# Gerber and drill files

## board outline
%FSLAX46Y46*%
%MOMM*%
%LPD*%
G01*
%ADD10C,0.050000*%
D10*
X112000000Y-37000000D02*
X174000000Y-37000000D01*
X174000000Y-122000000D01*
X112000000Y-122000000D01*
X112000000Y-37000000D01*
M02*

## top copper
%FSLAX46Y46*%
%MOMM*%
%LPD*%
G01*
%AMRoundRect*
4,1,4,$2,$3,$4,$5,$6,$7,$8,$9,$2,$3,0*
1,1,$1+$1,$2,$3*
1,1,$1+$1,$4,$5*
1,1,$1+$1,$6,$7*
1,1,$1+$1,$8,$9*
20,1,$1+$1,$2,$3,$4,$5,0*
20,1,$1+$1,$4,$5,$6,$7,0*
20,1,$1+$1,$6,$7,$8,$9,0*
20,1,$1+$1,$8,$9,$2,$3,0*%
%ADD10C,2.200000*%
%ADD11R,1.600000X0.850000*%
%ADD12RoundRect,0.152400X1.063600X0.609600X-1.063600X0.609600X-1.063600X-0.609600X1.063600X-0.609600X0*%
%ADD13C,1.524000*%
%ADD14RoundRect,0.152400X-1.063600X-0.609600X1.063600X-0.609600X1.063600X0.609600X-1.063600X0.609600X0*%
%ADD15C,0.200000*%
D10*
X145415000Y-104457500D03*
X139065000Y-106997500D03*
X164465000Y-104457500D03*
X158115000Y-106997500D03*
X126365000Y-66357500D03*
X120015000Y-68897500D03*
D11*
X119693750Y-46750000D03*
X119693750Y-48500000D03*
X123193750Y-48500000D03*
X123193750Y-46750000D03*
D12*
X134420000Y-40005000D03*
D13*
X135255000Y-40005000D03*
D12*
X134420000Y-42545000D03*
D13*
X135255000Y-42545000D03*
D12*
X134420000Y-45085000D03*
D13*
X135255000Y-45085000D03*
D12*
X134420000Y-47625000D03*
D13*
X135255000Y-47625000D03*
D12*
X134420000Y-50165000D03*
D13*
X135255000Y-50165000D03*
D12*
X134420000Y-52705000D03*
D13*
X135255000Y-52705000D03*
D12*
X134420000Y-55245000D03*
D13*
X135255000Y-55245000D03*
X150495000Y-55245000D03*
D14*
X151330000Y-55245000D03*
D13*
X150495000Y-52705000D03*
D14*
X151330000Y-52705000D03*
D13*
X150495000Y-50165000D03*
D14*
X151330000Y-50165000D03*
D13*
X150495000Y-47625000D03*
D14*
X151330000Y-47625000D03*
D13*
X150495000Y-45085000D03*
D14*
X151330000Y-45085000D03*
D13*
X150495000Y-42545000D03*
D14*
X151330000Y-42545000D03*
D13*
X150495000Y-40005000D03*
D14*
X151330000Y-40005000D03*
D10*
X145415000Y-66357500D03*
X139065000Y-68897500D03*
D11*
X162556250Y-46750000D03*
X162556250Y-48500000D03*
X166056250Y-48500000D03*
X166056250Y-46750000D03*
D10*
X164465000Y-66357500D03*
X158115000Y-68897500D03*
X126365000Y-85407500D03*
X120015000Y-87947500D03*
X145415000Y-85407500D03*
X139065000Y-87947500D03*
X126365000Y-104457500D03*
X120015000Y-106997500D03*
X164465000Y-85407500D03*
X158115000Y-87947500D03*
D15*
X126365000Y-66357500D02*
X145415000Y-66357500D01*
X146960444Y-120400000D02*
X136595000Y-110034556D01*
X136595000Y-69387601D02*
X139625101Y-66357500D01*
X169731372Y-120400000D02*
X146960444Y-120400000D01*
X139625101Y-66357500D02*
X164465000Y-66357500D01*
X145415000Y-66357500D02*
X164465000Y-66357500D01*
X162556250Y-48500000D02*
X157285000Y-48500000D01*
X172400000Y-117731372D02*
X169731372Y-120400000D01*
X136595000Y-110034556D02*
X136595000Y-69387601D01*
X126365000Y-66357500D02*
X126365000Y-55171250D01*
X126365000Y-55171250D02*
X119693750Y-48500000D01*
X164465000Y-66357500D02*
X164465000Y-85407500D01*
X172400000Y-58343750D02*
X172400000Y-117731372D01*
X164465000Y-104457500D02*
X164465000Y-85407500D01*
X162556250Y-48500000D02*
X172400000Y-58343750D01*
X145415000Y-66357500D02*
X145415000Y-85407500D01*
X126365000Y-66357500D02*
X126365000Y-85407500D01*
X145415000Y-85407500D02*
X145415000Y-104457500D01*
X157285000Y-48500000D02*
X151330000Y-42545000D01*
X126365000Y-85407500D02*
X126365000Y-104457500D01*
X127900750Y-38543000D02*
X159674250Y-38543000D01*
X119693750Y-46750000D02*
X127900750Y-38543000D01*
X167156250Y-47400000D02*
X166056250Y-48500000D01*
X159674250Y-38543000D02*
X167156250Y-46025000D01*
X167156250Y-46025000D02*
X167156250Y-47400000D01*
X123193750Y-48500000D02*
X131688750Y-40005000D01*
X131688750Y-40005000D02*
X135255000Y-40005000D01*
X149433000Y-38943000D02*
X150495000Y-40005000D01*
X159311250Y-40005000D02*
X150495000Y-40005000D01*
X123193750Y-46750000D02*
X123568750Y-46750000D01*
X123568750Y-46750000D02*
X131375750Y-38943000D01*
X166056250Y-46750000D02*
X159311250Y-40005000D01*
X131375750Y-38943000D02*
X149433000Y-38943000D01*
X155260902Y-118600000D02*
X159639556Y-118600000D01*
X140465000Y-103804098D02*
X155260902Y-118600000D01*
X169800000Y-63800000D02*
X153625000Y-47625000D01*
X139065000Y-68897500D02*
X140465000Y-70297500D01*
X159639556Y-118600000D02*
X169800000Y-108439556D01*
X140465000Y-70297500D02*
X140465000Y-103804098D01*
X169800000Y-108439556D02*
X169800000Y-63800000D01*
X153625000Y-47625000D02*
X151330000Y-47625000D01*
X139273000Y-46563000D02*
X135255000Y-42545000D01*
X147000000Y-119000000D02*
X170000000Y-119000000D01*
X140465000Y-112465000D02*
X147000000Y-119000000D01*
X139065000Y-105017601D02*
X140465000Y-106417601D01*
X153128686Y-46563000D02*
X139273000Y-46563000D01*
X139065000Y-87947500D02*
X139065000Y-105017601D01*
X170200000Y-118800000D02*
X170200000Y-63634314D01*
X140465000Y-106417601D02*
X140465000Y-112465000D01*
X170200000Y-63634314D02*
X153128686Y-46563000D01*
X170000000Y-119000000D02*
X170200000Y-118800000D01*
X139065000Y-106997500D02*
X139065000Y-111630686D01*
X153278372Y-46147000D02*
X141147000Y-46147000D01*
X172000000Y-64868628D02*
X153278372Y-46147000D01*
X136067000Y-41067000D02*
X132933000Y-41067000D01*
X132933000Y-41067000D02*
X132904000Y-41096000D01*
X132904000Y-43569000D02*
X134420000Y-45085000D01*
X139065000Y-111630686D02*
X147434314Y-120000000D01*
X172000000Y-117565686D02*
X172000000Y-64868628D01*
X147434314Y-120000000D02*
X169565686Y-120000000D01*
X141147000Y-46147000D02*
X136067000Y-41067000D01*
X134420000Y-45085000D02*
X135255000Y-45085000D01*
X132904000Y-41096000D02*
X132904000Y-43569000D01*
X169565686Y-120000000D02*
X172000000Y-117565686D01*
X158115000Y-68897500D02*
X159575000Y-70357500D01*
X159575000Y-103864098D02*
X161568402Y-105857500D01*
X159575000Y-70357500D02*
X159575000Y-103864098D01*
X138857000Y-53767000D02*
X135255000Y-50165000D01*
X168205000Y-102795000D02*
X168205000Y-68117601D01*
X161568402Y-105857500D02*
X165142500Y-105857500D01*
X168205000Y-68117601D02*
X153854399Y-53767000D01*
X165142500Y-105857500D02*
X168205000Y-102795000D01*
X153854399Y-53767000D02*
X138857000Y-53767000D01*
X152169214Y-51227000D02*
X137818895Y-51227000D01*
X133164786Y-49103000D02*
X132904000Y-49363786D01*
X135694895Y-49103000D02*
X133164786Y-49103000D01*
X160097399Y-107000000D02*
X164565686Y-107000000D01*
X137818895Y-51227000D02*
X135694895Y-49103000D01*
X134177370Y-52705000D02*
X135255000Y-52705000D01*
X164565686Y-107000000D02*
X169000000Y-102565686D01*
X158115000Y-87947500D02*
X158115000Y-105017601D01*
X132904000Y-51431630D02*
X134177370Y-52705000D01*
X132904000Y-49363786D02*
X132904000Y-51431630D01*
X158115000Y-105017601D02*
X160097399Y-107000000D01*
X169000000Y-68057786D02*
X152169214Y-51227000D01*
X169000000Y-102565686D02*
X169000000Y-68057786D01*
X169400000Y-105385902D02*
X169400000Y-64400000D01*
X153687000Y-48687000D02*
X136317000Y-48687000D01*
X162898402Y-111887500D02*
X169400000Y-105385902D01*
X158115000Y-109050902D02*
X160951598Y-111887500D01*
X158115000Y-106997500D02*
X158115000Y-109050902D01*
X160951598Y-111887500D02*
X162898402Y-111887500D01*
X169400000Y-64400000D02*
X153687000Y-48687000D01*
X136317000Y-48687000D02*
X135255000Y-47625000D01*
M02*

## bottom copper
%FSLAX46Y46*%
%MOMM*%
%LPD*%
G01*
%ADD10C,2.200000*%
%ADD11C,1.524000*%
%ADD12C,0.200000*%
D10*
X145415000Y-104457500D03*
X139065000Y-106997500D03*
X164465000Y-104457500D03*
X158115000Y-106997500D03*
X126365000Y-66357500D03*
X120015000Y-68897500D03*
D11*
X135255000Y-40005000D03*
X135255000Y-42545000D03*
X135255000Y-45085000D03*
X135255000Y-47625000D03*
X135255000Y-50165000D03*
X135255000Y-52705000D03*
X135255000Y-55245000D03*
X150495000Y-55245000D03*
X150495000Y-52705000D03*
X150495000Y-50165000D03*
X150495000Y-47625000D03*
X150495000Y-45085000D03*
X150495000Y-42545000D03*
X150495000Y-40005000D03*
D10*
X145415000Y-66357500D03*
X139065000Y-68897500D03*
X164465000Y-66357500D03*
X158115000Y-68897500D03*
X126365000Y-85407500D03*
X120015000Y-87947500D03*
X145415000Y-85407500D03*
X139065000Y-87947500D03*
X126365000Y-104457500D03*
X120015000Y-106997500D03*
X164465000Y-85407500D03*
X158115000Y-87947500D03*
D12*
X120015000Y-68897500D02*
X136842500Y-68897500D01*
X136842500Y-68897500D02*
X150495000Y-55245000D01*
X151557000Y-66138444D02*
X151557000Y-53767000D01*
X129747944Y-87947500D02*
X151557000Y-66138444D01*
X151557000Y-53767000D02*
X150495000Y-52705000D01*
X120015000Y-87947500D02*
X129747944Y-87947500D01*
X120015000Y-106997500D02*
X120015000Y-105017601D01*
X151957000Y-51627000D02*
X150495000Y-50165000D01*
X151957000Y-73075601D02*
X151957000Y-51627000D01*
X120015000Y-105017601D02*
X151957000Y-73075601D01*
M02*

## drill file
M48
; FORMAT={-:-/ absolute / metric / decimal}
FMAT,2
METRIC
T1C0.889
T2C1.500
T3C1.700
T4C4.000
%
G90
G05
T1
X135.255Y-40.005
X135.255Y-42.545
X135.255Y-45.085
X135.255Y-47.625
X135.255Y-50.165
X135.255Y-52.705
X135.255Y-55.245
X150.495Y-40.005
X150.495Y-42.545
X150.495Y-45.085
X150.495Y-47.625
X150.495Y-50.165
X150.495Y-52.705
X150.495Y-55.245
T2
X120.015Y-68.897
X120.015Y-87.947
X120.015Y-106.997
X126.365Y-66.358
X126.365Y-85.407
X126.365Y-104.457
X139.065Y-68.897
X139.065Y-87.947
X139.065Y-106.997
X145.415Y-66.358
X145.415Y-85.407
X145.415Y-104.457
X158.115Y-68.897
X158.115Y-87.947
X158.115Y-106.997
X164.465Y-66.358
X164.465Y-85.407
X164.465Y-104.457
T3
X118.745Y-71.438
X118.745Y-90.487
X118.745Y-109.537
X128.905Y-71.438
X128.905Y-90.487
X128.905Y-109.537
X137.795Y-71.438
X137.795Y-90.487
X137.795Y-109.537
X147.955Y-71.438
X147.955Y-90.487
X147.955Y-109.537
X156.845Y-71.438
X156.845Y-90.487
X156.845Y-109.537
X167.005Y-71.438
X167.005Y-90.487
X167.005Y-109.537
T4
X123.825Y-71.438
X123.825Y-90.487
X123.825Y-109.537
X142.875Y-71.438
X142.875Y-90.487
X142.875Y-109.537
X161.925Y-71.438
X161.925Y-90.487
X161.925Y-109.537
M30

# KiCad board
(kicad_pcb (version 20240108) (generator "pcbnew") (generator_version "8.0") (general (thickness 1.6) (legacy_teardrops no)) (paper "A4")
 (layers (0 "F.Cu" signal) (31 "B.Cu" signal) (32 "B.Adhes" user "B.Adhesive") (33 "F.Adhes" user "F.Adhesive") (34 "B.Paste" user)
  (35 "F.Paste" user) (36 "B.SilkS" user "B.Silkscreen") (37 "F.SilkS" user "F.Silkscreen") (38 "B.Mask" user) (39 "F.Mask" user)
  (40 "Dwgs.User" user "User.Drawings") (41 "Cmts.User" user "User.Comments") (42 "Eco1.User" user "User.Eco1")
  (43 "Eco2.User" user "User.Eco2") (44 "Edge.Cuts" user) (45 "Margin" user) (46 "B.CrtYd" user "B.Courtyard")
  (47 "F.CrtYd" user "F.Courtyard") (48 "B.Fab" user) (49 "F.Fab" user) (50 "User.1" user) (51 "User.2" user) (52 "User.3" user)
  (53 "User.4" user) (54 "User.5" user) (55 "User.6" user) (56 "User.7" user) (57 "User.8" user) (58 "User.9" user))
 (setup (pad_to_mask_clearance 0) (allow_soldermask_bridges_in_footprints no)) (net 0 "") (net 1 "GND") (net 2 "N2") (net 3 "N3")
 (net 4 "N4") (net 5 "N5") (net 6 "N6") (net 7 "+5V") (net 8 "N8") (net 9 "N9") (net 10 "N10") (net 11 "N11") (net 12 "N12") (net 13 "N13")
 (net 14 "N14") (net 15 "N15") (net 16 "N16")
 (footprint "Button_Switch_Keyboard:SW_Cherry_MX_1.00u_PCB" (layer "F.Cu") (at 145.415 104.4575)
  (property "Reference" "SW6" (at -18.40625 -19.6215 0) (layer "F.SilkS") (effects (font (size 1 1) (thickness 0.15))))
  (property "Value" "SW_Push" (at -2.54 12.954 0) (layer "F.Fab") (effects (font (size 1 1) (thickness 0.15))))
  (pad "" np_thru_hole circle (at -7.62 5.08) (size 1.7 1.7) (drill 1.7) (layers "*.Cu" "*.Mask"))
  (pad "" np_thru_hole circle (at -2.54 5.08) (size 4 4) (drill 4) (layers "*.Cu" "*.Mask"))
  (pad "" np_thru_hole circle (at 2.54 5.08) (size 1.7 1.7) (drill 1.7) (layers "*.Cu" "*.Mask"))
  (pad "1" thru_hole circle (at 0 0) (size 2.2 2.2) (drill 1.5) (layers "*.Cu" "*.Mask") (remove_unused_layers no) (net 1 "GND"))
  (pad "2" thru_hole circle (at -6.35 2.54) (size 2.2 2.2) (drill 1.5) (layers "*.Cu" "*.Mask") (remove_unused_layers no) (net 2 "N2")))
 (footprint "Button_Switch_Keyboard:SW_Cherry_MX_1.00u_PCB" (layer "F.Cu") (at 164.465 104.4575)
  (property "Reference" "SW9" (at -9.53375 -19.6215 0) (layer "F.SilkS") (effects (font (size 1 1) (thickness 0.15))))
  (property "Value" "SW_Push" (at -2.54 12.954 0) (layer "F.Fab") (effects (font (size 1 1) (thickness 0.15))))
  (pad "" np_thru_hole circle (at -7.62 5.08) (size 1.7 1.7) (drill 1.7) (layers "*.Cu" "*.Mask"))
  (pad "" np_thru_hole circle (at -2.54 5.08) (size 4 4) (drill 4) (layers "*.Cu" "*.Mask"))
  (pad "" np_thru_hole circle (at 2.54 5.08) (size 1.7 1.7) (drill 1.7) (layers "*.Cu" "*.Mask"))
  (pad "1" thru_hole circle (at 0 0) (size 2.2 2.2) (drill 1.5) (layers "*.Cu" "*.Mask") (remove_unused_layers no) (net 1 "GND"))
  (pad "2" thru_hole circle (at -6.35 2.54) (size 2.2 2.2) (drill 1.5) (layers "*.Cu" "*.Mask") (remove_unused_layers no) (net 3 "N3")))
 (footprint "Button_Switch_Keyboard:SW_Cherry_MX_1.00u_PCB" (layer "F.Cu") (at 126.365 66.3575)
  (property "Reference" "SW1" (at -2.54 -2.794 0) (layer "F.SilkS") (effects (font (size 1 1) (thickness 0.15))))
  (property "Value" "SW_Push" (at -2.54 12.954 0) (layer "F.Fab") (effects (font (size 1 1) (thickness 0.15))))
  (pad "" np_thru_hole circle (at -7.62 5.08) (size 1.7 1.7) (drill 1.7) (layers "*.Cu" "*.Mask"))
  (pad "" np_thru_hole circle (at -2.54 5.08) (size 4 4) (drill 4) (layers "*.Cu" "*.Mask"))
  (pad "" np_thru_hole circle (at 2.54 5.08) (size 1.7 1.7) (drill 1.7) (layers "*.Cu" "*.Mask"))
  (pad "1" thru_hole circle (at 0 0) (size 2.2 2.2) (drill 1.5) (layers "*.Cu" "*.Mask") (remove_unused_layers no) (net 1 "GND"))
  (pad "2" thru_hole circle (at -6.35 2.54) (size 2.2 2.2) (drill 1.5) (layers "*.Cu" "*.Mask") (remove_unused_layers no) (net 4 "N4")))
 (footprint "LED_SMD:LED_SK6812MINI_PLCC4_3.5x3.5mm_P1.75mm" (layer "F.Cu") (at 121.44375 47.625)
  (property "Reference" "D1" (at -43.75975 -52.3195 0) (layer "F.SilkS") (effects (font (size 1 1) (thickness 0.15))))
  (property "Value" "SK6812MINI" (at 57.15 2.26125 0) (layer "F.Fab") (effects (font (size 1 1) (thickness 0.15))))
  (pad "1" smd rect (at -1.75 -0.875) (size 1.6 0.85) (layers "F.Cu" "F.Paste" "F.Mask") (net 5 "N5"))
  (pad "2" smd rect (at -1.75 0.875) (size 1.6 0.85) (layers "F.Cu" "F.Paste" "F.Mask") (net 1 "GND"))
  (pad "3" smd rect (at 1.75 0.875) (size 1.6 0.85) (layers "F.Cu" "F.Paste" "F.Mask") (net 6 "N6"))
  (pad "4" smd rect (at 1.75 -0.875) (size 1.6 0.85) (layers "F.Cu" "F.Paste" "F.Mask") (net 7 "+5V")))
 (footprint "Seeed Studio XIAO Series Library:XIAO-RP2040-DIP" (layer "F.Cu") (at 142.875 47.625)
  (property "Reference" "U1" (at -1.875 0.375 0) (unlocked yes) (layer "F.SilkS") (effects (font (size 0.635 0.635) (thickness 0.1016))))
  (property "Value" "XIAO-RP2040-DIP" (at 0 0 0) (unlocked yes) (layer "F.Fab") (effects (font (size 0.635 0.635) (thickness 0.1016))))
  (pad "1" smd roundrect (at -8.455 -7.62 180) (size 2.432 1.524) (layers "F.Cu" "F.Mask") (roundrect_rratio 0.1) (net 6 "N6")
   (thermal_bridge_angle 45))
  (pad "1" thru_hole circle (at -7.62 -7.62 180) (size 1.524 1.524) (drill 0.889) (layers "*.Cu" "*.Mask") (remove_unused_layers no)
   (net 6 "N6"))
  (pad "2" smd roundrect (at -8.455 -5.08 180) (size 2.432 1.524) (layers "F.Cu" "F.Mask") (roundrect_rratio 0.1) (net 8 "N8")
   (thermal_bridge_angle 45))
  (pad "2" thru_hole circle (at -7.62 -5.08 180) (size 1.524 1.524) (drill 0.889) (layers "*.Cu" "*.Mask") (remove_unused_layers no)
   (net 8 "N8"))
  (pad "3" smd roundrect (at -8.455 -2.54 180) (size 2.432 1.524) (layers "F.Cu" "F.Mask") (roundrect_rratio 0.1) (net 2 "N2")
   (thermal_bridge_angle 45))
  (pad "3" thru_hole circle (at -7.62 -2.54 180) (size 1.524 1.524) (drill 0.889) (layers "*.Cu" "*.Mask") (remove_unused_layers no)
   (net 2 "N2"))
  (pad "4" smd roundrect (at -8.455 0 180) (size 2.432 1.524) (layers "F.Cu" "F.Mask") (roundrect_rratio 0.1) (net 3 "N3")
   (thermal_bridge_angle 45))
  (pad "4" thru_hole circle (at -7.62 0 180) (size 1.524 1.524) (drill 0.889) (layers "*.Cu" "*.Mask") (remove_unused_layers no)
   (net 3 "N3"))
  (pad "5" smd roundrect (at -8.455 2.54 180) (size 2.432 1.524) (layers "F.Cu" "F.Mask") (roundrect_rratio 0.1) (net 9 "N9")
   (thermal_bridge_angle 45))
  (pad "5" thru_hole circle (at -7.62 2.54 180) (size 1.524 1.524) (drill 0.889) (layers "*.Cu" "*.Mask") (remove_unused_layers no)
   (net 9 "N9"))
  (pad "6" smd roundrect (at -8.455 5.08 180) (size 2.432 1.524) (layers "F.Cu" "F.Mask") (roundrect_rratio 0.1) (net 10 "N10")
   (thermal_bridge_angle 45))
  (pad "6" thru_hole circle (at -7.62 5.08 180) (size 1.524 1.524) (drill 0.889) (layers "*.Cu" "*.Mask") (remove_unused_layers no)
   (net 10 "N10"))
  (pad "7" smd roundrect (at -8.455 7.62 180) (size 2.432 1.524) (layers "F.Cu" "F.Mask") (roundrect_rratio 0.1) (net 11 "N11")
   (thermal_bridge_angle 45))
  (pad "7" thru_hole circle (at -7.62 7.62 180) (size 1.524 1.524) (drill 0.889) (layers "*.Cu" "*.Mask") (remove_unused_layers no)
   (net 11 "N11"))
  (pad "8" thru_hole circle (at 7.62 7.62) (size 1.524 1.524) (drill 0.889) (layers "*.Cu" "*.Mask") (remove_unused_layers no) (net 4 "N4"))
  (pad "8" smd roundrect (at 8.455 7.62) (size 2.432 1.524) (layers "F.Cu" "F.Mask") (roundrect_rratio 0.1) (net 4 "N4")
   (thermal_bridge_angle 45))
  (pad "9" thru_hole circle (at 7.62 5.08) (size 1.524 1.524) (drill 0.889) (layers "*.Cu" "*.Mask") (remove_unused_layers no)
   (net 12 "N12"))
  (pad "9" smd roundrect (at 8.455 5.08) (size 2.432 1.524) (layers "F.Cu" "F.Mask") (roundrect_rratio 0.1) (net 12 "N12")
   (thermal_bridge_angle 45))
  (pad "10" thru_hole circle (at 7.62 2.54) (size 1.524 1.524) (drill 0.889) (layers "*.Cu" "*.Mask") (remove_unused_layers no)
   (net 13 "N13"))
  (pad "10" smd roundrect (at 8.455 2.54) (size 2.432 1.524) (layers "F.Cu" "F.Mask") (roundrect_rratio 0.1) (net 13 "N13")
   (thermal_bridge_angle 45))
  (pad "11" thru_hole circle (at 7.62 0) (size 1.524 1.524) (drill 0.889) (layers "*.Cu" "*.Mask") (remove_unused_layers no) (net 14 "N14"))
  (pad "11" smd roundrect (at 8.455 0) (size 2.432 1.524) (layers "F.Cu" "F.Mask") (roundrect_rratio 0.1) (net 14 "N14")
   (thermal_bridge_angle 45))
  (pad "12" thru_hole circle (at 7.62 -2.54) (size 1.524 1.524) (drill 0.889) (layers "*.Cu" "*.Mask") (remove_unused_layers no)
   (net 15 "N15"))
  (pad "12" smd roundrect (at 8.455 -2.54) (size 2.432 1.524) (layers "F.Cu" "F.Mask") (roundrect_rratio 0.1) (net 15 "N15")
   (thermal_bridge_angle 45))
  (pad "13" thru_hole circle (at 7.62 -5.08) (size 1.524 1.524) (drill 0.889) (layers "*.Cu" "*.Mask") (remove_unused_layers no)
   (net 1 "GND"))
  (pad "13" smd roundrect (at 8.455 -5.08) (size 2.432 1.524) (layers "F.Cu" "F.Mask") (roundrect_rratio 0.1) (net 1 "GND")
   (thermal_bridge_angle 45))
  (pad "14" thru_hole circle (at 7.62 -7.62) (size 1.524 1.524) (drill 0.889) (layers "*.Cu" "*.Mask") (remove_unused_layers no)
   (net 7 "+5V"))
  (pad "14" smd roundrect (at 8.455 -7.62) (size 2.432 1.524) (layers "F.Cu" "F.Mask") (roundrect_rratio 0.1) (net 7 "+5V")
   (thermal_bridge_angle 45)))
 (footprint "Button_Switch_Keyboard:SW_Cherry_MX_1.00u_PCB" (layer "F.Cu") (at 145.415 66.3575)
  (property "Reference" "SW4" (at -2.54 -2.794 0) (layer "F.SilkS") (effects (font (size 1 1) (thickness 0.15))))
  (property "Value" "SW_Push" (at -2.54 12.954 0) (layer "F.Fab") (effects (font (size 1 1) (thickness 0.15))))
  (pad "" np_thru_hole circle (at -7.62 5.08) (size 1.7 1.7) (drill 1.7) (layers "*.Cu" "*.Mask"))
  (pad "" np_thru_hole circle (at -2.54 5.08) (size 4 4) (drill 4) (layers "*.Cu" "*.Mask"))
  (pad "" np_thru_hole circle (at 2.54 5.08) (size 1.7 1.7) (drill 1.7) (layers "*.Cu" "*.Mask"))
  (pad "1" thru_hole circle (at 0 0) (size 2.2 2.2) (drill 1.5) (layers "*.Cu" "*.Mask") (remove_unused_layers no) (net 1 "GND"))
  (pad "2" thru_hole circle (at -6.35 2.54) (size 2.2 2.2) (drill 1.5) (layers "*.Cu" "*.Mask") (remove_unused_layers no) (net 14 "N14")))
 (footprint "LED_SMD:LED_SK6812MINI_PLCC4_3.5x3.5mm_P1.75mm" (layer "F.Cu") (at 164.30625 47.625)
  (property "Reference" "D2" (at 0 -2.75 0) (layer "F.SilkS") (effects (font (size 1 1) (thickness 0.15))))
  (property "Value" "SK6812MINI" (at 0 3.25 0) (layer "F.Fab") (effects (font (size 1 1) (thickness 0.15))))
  (pad "1" smd rect (at -1.75 -0.875) (size 1.6 0.85) (layers "F.Cu" "F.Paste" "F.Mask") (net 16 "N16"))
  (pad "2" smd rect (at -1.75 0.875) (size 1.6 0.85) (layers "F.Cu" "F.Paste" "F.Mask") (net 1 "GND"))
  (pad "3" smd rect (at 1.75 0.875) (size 1.6 0.85) (layers "F.Cu" "F.Paste" "F.Mask") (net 5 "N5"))
  (pad "4" smd rect (at 1.75 -0.875) (size 1.6 0.85) (layers "F.Cu" "F.Paste" "F.Mask") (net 7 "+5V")))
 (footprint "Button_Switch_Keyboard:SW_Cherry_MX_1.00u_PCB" (layer "F.Cu") (at 164.465 66.3575)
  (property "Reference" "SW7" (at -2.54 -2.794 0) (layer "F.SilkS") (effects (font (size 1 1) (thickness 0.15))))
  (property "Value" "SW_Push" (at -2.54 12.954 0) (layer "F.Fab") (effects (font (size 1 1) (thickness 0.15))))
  (pad "" np_thru_hole circle (at -7.62 5.08) (size 1.7 1.7) (drill 1.7) (layers "*.Cu" "*.Mask"))
  (pad "" np_thru_hole circle (at -2.54 5.08) (size 4 4) (drill 4) (layers "*.Cu" "*.Mask"))
  (pad "" np_thru_hole circle (at 2.54 5.08) (size 1.7 1.7) (drill 1.7) (layers "*.Cu" "*.Mask"))
  (pad "1" thru_hole circle (at 0 0) (size 2.2 2.2) (drill 1.5) (layers "*.Cu" "*.Mask") (remove_unused_layers no) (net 1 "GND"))
  (pad "2" thru_hole circle (at -6.35 2.54) (size 2.2 2.2) (drill 1.5) (layers "*.Cu" "*.Mask") (remove_unused_layers no) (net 9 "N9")))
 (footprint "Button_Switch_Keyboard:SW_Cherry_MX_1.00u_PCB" (layer "F.Cu") (at 126.365 85.4075)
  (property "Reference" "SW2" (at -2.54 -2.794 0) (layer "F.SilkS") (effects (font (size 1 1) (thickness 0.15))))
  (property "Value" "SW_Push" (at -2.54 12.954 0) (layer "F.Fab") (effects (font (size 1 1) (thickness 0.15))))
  (pad "" np_thru_hole circle (at -7.62 5.08) (size 1.7 1.7) (drill 1.7) (layers "*.Cu" "*.Mask"))
  (pad "" np_thru_hole circle (at -2.54 5.08) (size 4 4) (drill 4) (layers "*.Cu" "*.Mask"))
  (pad "" np_thru_hole circle (at 2.54 5.08) (size 1.7 1.7) (drill 1.7) (layers "*.Cu" "*.Mask"))
  (pad "1" thru_hole circle (at 0 0) (size 2.2 2.2) (drill 1.5) (layers "*.Cu" "*.Mask") (remove_unused_layers no) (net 1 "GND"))
  (pad "2" thru_hole circle (at -6.35 2.54) (size 2.2 2.2) (drill 1.5) (layers "*.Cu" "*.Mask") (remove_unused_layers no) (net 12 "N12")))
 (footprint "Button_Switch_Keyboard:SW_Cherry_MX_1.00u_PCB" (layer "F.Cu") (at 145.415 85.4075)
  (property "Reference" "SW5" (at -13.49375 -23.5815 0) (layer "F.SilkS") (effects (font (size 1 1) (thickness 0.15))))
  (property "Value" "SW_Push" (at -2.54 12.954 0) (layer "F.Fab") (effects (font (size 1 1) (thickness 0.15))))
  (pad "" np_thru_hole circle (at -7.62 5.08) (size 1.7 1.7) (drill 1.7) (layers "*.Cu" "*.Mask"))
  (pad "" np_thru_hole circle (at -2.54 5.08) (size 4 4) (drill 4) (layers "*.Cu" "*.Mask"))
  (pad "" np_thru_hole circle (at 2.54 5.08) (size 1.7 1.7) (drill 1.7) (layers "*.Cu" "*.Mask"))
  (pad "1" thru_hole circle (at 0 0) (size 2.2 2.2) (drill 1.5) (layers "*.Cu" "*.Mask") (remove_unused_layers no) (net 1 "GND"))
  (pad "2" thru_hole circle (at -6.35 2.54) (size 2.2 2.2) (drill 1.5) (layers "*.Cu" "*.Mask") (remove_unused_layers no) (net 8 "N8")))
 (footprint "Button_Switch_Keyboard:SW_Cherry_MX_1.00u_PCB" (layer "F.Cu") (at 126.365 104.4575)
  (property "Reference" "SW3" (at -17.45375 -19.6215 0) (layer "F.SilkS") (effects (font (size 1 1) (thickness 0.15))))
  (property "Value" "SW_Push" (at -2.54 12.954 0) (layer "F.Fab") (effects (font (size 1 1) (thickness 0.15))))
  (pad "" np_thru_hole circle (at -7.62 5.08) (size 1.7 1.7) (drill 1.7) (layers "*.Cu" "*.Mask"))
  (pad "" np_thru_hole circle (at -2.54 5.08) (size 4 4) (drill 4) (layers "*.Cu" "*.Mask"))
  (pad "" np_thru_hole circle (at 2.54 5.08) (size 1.7 1.7) (drill 1.7) (layers "*.Cu" "*.Mask"))
  (pad "1" thru_hole circle (at 0 0) (size 2.2 2.2) (drill 1.5) (layers "*.Cu" "*.Mask") (remove_unused_layers no) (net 1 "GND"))
  (pad "2" thru_hole circle (at -6.35 2.54) (size 2.2 2.2) (drill 1.5) (layers "*.Cu" "*.Mask") (remove_unused_layers no) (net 13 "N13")))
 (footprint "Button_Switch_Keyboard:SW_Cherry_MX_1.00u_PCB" (layer "F.Cu") (at 164.465 85.4075)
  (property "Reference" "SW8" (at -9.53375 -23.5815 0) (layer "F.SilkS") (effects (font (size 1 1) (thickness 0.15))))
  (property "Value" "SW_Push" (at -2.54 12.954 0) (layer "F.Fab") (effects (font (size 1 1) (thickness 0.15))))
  (pad "" np_thru_hole circle (at -7.62 5.08) (size 1.7 1.7) (drill 1.7) (layers "*.Cu" "*.Mask"))
  (pad "" np_thru_hole circle (at -2.54 5.08) (size 4 4) (drill 4) (layers "*.Cu" "*.Mask"))
  (pad "" np_thru_hole circle (at 2.54 5.08) (size 1.7 1.7) (drill 1.7) (layers "*.Cu" "*.Mask"))
  (pad "1" thru_hole circle (at 0 0) (size 2.2 2.2) (drill 1.5) (layers "*.Cu" "*.Mask") (remove_unused_layers no) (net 1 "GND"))
  (pad "2" thru_hole circle (at -6.35 2.54) (size 2.2 2.2) (drill 1.5) (layers "*.Cu" "*.Mask") (remove_unused_layers no) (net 10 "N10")))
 (gr_rect (start 112 37) (end 174 122) (stroke (width 0.05) (type default)) (fill none) (layer "Edge.Cuts"))
 (segment (start 126.365 66.3575) (end 145.415 66.3575) (width 0.2) (layer "F.Cu") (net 1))
 (segment (start 146.960444 120.4) (end 136.595 110.034556) (width 0.2) (layer "F.Cu") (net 1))
 (segment (start 136.595 69.387601) (end 139.625101 66.3575) (width 0.2) (layer "F.Cu") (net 1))
 (segment (start 169.731372 120.4) (end 146.960444 120.4) (width 0.2) (layer "F.Cu") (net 1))
 (segment (start 139.625101 66.3575) (end 164.465 66.3575) (width 0.2) (layer "F.Cu") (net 1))
 (segment (start 145.415 66.3575) (end 164.465 66.3575) (width 0.2) (layer "F.Cu") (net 1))
 (segment (start 162.55625 48.5) (end 157.285 48.5) (width 0.2) (layer "F.Cu") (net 1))
 (segment (start 172.4 117.731372) (end 169.731372 120.4) (width 0.2) (layer "F.Cu") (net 1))
 (segment (start 136.595 110.034556) (end 136.595 69.387601) (width 0.2) (layer "F.Cu") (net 1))
 (segment (start 126.365 66.3575) (end 126.365 55.17125) (width 0.2) (layer "F.Cu") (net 1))
 (segment (start 126.365 55.17125) (end 119.69375 48.5) (width 0.2) (layer "F.Cu") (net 1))
 (segment (start 164.465 66.3575) (end 164.465 85.4075) (width 0.2) (layer "F.Cu") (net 1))
 (segment (start 172.4 58.34375) (end 172.4 117.731372) (width 0.2) (layer "F.Cu") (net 1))
 (segment (start 164.465 104.4575) (end 164.465 85.4075) (width 0.2) (layer "F.Cu") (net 1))
 (segment (start 162.55625 48.5) (end 172.4 58.34375) (width 0.2) (layer "F.Cu") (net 1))
 (segment (start 145.415 66.3575) (end 145.415 85.4075) (width 0.2) (layer "F.Cu") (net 1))
 (segment (start 126.365 66.3575) (end 126.365 85.4075) (width 0.2) (layer "F.Cu") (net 1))
 (segment (start 145.415 85.4075) (end 145.415 104.4575) (width 0.2) (layer "F.Cu") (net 1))
 (segment (start 157.285 48.5) (end 151.33 42.545) (width 0.2) (layer "F.Cu") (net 1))
 (segment (start 126.365 85.4075) (end 126.365 104.4575) (width 0.2) (layer "F.Cu") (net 1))
 (segment (start 127.90075 38.543) (end 159.67425 38.543) (width 0.2) (layer "F.Cu") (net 5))
 (segment (start 119.69375 46.75) (end 127.90075 38.543) (width 0.2) (layer "F.Cu") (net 5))
 (segment (start 167.15625 47.4) (end 166.05625 48.5) (width 0.2) (layer "F.Cu") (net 5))
 (segment (start 159.67425 38.543) (end 167.15625 46.025) (width 0.2) (layer "F.Cu") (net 5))
 (segment (start 167.15625 46.025) (end 167.15625 47.4) (width 0.2) (layer "F.Cu") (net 5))
 (segment (start 123.19375 48.5) (end 131.68875 40.005) (width 0.2) (layer "F.Cu") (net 6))
 (segment (start 131.68875 40.005) (end 135.255 40.005) (width 0.2) (layer "F.Cu") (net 6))
 (segment (start 149.433 38.943) (end 150.495 40.005) (width 0.2) (layer "F.Cu") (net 7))
 (segment (start 159.31125 40.005) (end 150.495 40.005) (width 0.2) (layer "F.Cu") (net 7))
 (segment (start 123.19375 46.75) (end 123.56875 46.75) (width 0.2) (layer "F.Cu") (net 7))
 (segment (start 123.56875 46.75) (end 131.37575 38.943) (width 0.2) (layer "F.Cu") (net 7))
 (segment (start 166.05625 46.75) (end 159.31125 40.005) (width 0.2) (layer "F.Cu") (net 7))
 (segment (start 131.37575 38.943) (end 149.433 38.943) (width 0.2) (layer "F.Cu") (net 7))
 (segment (start 120.015 68.8975) (end 136.8425 68.8975) (width 0.2) (layer "B.Cu") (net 4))
 (segment (start 136.8425 68.8975) (end 150.495 55.245) (width 0.2) (layer "B.Cu") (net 4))
 (segment (start 151.557 66.138444) (end 151.557 53.767) (width 0.2) (layer "B.Cu") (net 12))
 (segment (start 129.747944 87.9475) (end 151.557 66.138444) (width 0.2) (layer "B.Cu") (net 12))
 (segment (start 151.557 53.767) (end 150.495 52.705) (width 0.2) (layer "B.Cu") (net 12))
 (segment (start 120.015 87.9475) (end 129.747944 87.9475) (width 0.2) (layer "B.Cu") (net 12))
 (segment (start 120.015 106.9975) (end 120.015 105.017601) (width 0.2) (layer "B.Cu") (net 13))
 (segment (start 151.957 51.627) (end 150.495 50.165) (width 0.2) (layer "B.Cu") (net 13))
 (segment (start 151.957 73.075601) (end 151.957 51.627) (width 0.2) (layer "B.Cu") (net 13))
 (segment (start 120.015 105.017601) (end 151.957 73.075601) (width 0.2) (layer "B.Cu") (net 13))
 (segment (start 155.260902 118.6) (end 159.639556 118.6) (width 0.2) (layer "F.Cu") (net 14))
 (segment (start 140.465 103.804098) (end 155.260902 118.6) (width 0.2) (layer "F.Cu") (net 14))
 (segment (start 169.8 63.8) (end 153.625 47.625) (width 0.2) (layer "F.Cu") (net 14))
 (segment (start 139.065 68.8975) (end 140.465 70.2975) (width 0.2) (layer "F.Cu") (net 14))
 (segment (start 159.639556 118.6) (end 169.8 108.439556) (width 0.2) (layer "F.Cu") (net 14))
 (segment (start 140.465 70.2975) (end 140.465 103.804098) (width 0.2) (layer "F.Cu") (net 14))
 (segment (start 169.8 108.439556) (end 169.8 63.8) (width 0.2) (layer "F.Cu") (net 14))
 (segment (start 153.625 47.625) (end 151.33 47.625) (width 0.2) (layer "F.Cu") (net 14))
 (segment (start 139.273 46.563) (end 135.255 42.545) (width 0.2) (layer "F.Cu") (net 8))
 (segment (start 147 119) (end 170 119) (width 0.2) (layer "F.Cu") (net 8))
 (segment (start 140.465 112.465) (end 147 119) (width 0.2) (layer "F.Cu") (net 8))
 (segment (start 139.065 105.017601) (end 140.465 106.417601) (width 0.2) (layer "F.Cu") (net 8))
 (segment (start 153.128686 46.563) (end 139.273 46.563) (width 0.2) (layer "F.Cu") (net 8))
 (segment (start 139.065 87.9475) (end 139.065 105.017601) (width 0.2) (layer "F.Cu") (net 8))
 (segment (start 170.2 118.8) (end 170.2 63.634314) (width 0.2) (layer "F.Cu") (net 8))
 (segment (start 140.465 106.417601) (end 140.465 112.465) (width 0.2) (layer "F.Cu") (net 8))
 (segment (start 170.2 63.634314) (end 153.128686 46.563) (width 0.2) (layer "F.Cu") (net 8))
 (segment (start 170 119) (end 170.2 118.8) (width 0.2) (layer "F.Cu") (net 8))
 (segment (start 139.065 106.9975) (end 139.065 111.630686) (width 0.2) (layer "F.Cu") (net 2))
 (segment (start 153.278372 46.147) (end 141.147 46.147) (width 0.2) (layer "F.Cu") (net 2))
 (segment (start 172 64.868628) (end 153.278372 46.147) (width 0.2) (layer "F.Cu") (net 2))
 (segment (start 136.067 41.067) (end 132.933 41.067) (width 0.2) (layer "F.Cu") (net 2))
 (segment (start 132.933 41.067) (end 132.904 41.096) (width 0.2) (layer "F.Cu") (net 2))
 (segment (start 132.904 43.569) (end 134.42 45.085) (width 0.2) (layer "F.Cu") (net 2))
 (segment (start 139.065 111.630686) (end 147.434314 120) (width 0.2) (layer "F.Cu") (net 2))
 (segment (start 172 117.565686) (end 172 64.868628) (width 0.2) (layer "F.Cu") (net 2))
 (segment (start 147.434314 120) (end 169.565686 120) (width 0.2) (layer "F.Cu") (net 2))
 (segment (start 141.147 46.147) (end 136.067 41.067) (width 0.2) (layer "F.Cu") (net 2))
 (segment (start 134.42 45.085) (end 135.255 45.085) (width 0.2) (layer "F.Cu") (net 2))
 (segment (start 132.904 41.096) (end 132.904 43.569) (width 0.2) (layer "F.Cu") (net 2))
 (segment (start 169.565686 120) (end 172 117.565686) (width 0.2) (layer "F.Cu") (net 2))
 (segment (start 158.115 68.8975) (end 159.575 70.3575) (width 0.2) (layer "F.Cu") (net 9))
 (segment (start 159.575 103.864098) (end 161.568402 105.8575) (width 0.2) (layer "F.Cu") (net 9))
 (segment (start 159.575 70.3575) (end 159.575 103.864098) (width 0.2) (layer "F.Cu") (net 9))
 (segment (start 138.857 53.767) (end 135.255 50.165) (width 0.2) (layer "F.Cu") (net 9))
 (segment (start 168.205 102.795) (end 168.205 68.117601) (width 0.2) (layer "F.Cu") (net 9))
 (segment (start 161.568402 105.8575) (end 165.1425 105.8575) (width 0.2) (layer "F.Cu") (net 9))
 (segment (start 168.205 68.117601) (end 153.854399 53.767) (width 0.2) (layer "F.Cu") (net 9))
 (segment (start 165.1425 105.8575) (end 168.205 102.795) (width 0.2) (layer "F.Cu") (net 9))
 (segment (start 153.854399 53.767) (end 138.857 53.767) (width 0.2) (layer "F.Cu") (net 9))
 (segment (start 152.169214 51.227) (end 137.818895 51.227) (width 0.2) (layer "F.Cu") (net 10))
 (segment (start 133.164786 49.103) (end 132.904 49.363786) (width 0.2) (layer "F.Cu") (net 10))
 (segment (start 135.694895 49.103) (end 133.164786 49.103) (width 0.2) (layer "F.Cu") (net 10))
 (segment (start 160.097399 107) (end 164.565686 107) (width 0.2) (layer "F.Cu") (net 10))
 (segment (start 137.818895 51.227) (end 135.694895 49.103) (width 0.2) (layer "F.Cu") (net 10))
 (segment (start 134.17737 52.705) (end 135.255 52.705) (width 0.2) (layer "F.Cu") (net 10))
 (segment (start 164.565686 107) (end 169 102.565686) (width 0.2) (layer "F.Cu") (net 10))
 (segment (start 158.115 87.9475) (end 158.115 105.017601) (width 0.2) (layer "F.Cu") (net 10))
 (segment (start 132.904 51.43163) (end 134.17737 52.705) (width 0.2) (layer "F.Cu") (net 10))
 (segment (start 132.904 49.363786) (end 132.904 51.43163) (width 0.2) (layer "F.Cu") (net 10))
 (segment (start 158.115 105.017601) (end 160.097399 107) (width 0.2) (layer "F.Cu") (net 10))
 (segment (start 169 68.057786) (end 152.169214 51.227) (width 0.2) (layer "F.Cu") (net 10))
 (segment (start 169 102.565686) (end 169 68.057786) (width 0.2) (layer "F.Cu") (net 10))
 (segment (start 169.4 105.385902) (end 169.4 64.4) (width 0.2) (layer "F.Cu") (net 3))
 (segment (start 153.687 48.687) (end 136.317 48.687) (width 0.2) (layer "F.Cu") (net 3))
 (segment (start 162.898402 111.8875) (end 169.4 105.385902) (width 0.2) (layer "F.Cu") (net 3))
 (segment (start 158.115 109.050902) (end 160.951598 111.8875) (width 0.2) (layer "F.Cu") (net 3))
 (segment (start 158.115 106.9975) (end 158.115 109.050902) (width 0.2) (layer "F.Cu") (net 3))
 (segment (start 160.951598 111.8875) (end 162.898402 111.8875) (width 0.2) (layer "F.Cu") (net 3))
 (segment (start 169.4 64.4) (end 153.687 48.687) (width 0.2) (layer "F.Cu") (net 3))
 (segment (start 136.317 48.687) (end 135.255 47.625) (width 0.2) (layer "F.Cu") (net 3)))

